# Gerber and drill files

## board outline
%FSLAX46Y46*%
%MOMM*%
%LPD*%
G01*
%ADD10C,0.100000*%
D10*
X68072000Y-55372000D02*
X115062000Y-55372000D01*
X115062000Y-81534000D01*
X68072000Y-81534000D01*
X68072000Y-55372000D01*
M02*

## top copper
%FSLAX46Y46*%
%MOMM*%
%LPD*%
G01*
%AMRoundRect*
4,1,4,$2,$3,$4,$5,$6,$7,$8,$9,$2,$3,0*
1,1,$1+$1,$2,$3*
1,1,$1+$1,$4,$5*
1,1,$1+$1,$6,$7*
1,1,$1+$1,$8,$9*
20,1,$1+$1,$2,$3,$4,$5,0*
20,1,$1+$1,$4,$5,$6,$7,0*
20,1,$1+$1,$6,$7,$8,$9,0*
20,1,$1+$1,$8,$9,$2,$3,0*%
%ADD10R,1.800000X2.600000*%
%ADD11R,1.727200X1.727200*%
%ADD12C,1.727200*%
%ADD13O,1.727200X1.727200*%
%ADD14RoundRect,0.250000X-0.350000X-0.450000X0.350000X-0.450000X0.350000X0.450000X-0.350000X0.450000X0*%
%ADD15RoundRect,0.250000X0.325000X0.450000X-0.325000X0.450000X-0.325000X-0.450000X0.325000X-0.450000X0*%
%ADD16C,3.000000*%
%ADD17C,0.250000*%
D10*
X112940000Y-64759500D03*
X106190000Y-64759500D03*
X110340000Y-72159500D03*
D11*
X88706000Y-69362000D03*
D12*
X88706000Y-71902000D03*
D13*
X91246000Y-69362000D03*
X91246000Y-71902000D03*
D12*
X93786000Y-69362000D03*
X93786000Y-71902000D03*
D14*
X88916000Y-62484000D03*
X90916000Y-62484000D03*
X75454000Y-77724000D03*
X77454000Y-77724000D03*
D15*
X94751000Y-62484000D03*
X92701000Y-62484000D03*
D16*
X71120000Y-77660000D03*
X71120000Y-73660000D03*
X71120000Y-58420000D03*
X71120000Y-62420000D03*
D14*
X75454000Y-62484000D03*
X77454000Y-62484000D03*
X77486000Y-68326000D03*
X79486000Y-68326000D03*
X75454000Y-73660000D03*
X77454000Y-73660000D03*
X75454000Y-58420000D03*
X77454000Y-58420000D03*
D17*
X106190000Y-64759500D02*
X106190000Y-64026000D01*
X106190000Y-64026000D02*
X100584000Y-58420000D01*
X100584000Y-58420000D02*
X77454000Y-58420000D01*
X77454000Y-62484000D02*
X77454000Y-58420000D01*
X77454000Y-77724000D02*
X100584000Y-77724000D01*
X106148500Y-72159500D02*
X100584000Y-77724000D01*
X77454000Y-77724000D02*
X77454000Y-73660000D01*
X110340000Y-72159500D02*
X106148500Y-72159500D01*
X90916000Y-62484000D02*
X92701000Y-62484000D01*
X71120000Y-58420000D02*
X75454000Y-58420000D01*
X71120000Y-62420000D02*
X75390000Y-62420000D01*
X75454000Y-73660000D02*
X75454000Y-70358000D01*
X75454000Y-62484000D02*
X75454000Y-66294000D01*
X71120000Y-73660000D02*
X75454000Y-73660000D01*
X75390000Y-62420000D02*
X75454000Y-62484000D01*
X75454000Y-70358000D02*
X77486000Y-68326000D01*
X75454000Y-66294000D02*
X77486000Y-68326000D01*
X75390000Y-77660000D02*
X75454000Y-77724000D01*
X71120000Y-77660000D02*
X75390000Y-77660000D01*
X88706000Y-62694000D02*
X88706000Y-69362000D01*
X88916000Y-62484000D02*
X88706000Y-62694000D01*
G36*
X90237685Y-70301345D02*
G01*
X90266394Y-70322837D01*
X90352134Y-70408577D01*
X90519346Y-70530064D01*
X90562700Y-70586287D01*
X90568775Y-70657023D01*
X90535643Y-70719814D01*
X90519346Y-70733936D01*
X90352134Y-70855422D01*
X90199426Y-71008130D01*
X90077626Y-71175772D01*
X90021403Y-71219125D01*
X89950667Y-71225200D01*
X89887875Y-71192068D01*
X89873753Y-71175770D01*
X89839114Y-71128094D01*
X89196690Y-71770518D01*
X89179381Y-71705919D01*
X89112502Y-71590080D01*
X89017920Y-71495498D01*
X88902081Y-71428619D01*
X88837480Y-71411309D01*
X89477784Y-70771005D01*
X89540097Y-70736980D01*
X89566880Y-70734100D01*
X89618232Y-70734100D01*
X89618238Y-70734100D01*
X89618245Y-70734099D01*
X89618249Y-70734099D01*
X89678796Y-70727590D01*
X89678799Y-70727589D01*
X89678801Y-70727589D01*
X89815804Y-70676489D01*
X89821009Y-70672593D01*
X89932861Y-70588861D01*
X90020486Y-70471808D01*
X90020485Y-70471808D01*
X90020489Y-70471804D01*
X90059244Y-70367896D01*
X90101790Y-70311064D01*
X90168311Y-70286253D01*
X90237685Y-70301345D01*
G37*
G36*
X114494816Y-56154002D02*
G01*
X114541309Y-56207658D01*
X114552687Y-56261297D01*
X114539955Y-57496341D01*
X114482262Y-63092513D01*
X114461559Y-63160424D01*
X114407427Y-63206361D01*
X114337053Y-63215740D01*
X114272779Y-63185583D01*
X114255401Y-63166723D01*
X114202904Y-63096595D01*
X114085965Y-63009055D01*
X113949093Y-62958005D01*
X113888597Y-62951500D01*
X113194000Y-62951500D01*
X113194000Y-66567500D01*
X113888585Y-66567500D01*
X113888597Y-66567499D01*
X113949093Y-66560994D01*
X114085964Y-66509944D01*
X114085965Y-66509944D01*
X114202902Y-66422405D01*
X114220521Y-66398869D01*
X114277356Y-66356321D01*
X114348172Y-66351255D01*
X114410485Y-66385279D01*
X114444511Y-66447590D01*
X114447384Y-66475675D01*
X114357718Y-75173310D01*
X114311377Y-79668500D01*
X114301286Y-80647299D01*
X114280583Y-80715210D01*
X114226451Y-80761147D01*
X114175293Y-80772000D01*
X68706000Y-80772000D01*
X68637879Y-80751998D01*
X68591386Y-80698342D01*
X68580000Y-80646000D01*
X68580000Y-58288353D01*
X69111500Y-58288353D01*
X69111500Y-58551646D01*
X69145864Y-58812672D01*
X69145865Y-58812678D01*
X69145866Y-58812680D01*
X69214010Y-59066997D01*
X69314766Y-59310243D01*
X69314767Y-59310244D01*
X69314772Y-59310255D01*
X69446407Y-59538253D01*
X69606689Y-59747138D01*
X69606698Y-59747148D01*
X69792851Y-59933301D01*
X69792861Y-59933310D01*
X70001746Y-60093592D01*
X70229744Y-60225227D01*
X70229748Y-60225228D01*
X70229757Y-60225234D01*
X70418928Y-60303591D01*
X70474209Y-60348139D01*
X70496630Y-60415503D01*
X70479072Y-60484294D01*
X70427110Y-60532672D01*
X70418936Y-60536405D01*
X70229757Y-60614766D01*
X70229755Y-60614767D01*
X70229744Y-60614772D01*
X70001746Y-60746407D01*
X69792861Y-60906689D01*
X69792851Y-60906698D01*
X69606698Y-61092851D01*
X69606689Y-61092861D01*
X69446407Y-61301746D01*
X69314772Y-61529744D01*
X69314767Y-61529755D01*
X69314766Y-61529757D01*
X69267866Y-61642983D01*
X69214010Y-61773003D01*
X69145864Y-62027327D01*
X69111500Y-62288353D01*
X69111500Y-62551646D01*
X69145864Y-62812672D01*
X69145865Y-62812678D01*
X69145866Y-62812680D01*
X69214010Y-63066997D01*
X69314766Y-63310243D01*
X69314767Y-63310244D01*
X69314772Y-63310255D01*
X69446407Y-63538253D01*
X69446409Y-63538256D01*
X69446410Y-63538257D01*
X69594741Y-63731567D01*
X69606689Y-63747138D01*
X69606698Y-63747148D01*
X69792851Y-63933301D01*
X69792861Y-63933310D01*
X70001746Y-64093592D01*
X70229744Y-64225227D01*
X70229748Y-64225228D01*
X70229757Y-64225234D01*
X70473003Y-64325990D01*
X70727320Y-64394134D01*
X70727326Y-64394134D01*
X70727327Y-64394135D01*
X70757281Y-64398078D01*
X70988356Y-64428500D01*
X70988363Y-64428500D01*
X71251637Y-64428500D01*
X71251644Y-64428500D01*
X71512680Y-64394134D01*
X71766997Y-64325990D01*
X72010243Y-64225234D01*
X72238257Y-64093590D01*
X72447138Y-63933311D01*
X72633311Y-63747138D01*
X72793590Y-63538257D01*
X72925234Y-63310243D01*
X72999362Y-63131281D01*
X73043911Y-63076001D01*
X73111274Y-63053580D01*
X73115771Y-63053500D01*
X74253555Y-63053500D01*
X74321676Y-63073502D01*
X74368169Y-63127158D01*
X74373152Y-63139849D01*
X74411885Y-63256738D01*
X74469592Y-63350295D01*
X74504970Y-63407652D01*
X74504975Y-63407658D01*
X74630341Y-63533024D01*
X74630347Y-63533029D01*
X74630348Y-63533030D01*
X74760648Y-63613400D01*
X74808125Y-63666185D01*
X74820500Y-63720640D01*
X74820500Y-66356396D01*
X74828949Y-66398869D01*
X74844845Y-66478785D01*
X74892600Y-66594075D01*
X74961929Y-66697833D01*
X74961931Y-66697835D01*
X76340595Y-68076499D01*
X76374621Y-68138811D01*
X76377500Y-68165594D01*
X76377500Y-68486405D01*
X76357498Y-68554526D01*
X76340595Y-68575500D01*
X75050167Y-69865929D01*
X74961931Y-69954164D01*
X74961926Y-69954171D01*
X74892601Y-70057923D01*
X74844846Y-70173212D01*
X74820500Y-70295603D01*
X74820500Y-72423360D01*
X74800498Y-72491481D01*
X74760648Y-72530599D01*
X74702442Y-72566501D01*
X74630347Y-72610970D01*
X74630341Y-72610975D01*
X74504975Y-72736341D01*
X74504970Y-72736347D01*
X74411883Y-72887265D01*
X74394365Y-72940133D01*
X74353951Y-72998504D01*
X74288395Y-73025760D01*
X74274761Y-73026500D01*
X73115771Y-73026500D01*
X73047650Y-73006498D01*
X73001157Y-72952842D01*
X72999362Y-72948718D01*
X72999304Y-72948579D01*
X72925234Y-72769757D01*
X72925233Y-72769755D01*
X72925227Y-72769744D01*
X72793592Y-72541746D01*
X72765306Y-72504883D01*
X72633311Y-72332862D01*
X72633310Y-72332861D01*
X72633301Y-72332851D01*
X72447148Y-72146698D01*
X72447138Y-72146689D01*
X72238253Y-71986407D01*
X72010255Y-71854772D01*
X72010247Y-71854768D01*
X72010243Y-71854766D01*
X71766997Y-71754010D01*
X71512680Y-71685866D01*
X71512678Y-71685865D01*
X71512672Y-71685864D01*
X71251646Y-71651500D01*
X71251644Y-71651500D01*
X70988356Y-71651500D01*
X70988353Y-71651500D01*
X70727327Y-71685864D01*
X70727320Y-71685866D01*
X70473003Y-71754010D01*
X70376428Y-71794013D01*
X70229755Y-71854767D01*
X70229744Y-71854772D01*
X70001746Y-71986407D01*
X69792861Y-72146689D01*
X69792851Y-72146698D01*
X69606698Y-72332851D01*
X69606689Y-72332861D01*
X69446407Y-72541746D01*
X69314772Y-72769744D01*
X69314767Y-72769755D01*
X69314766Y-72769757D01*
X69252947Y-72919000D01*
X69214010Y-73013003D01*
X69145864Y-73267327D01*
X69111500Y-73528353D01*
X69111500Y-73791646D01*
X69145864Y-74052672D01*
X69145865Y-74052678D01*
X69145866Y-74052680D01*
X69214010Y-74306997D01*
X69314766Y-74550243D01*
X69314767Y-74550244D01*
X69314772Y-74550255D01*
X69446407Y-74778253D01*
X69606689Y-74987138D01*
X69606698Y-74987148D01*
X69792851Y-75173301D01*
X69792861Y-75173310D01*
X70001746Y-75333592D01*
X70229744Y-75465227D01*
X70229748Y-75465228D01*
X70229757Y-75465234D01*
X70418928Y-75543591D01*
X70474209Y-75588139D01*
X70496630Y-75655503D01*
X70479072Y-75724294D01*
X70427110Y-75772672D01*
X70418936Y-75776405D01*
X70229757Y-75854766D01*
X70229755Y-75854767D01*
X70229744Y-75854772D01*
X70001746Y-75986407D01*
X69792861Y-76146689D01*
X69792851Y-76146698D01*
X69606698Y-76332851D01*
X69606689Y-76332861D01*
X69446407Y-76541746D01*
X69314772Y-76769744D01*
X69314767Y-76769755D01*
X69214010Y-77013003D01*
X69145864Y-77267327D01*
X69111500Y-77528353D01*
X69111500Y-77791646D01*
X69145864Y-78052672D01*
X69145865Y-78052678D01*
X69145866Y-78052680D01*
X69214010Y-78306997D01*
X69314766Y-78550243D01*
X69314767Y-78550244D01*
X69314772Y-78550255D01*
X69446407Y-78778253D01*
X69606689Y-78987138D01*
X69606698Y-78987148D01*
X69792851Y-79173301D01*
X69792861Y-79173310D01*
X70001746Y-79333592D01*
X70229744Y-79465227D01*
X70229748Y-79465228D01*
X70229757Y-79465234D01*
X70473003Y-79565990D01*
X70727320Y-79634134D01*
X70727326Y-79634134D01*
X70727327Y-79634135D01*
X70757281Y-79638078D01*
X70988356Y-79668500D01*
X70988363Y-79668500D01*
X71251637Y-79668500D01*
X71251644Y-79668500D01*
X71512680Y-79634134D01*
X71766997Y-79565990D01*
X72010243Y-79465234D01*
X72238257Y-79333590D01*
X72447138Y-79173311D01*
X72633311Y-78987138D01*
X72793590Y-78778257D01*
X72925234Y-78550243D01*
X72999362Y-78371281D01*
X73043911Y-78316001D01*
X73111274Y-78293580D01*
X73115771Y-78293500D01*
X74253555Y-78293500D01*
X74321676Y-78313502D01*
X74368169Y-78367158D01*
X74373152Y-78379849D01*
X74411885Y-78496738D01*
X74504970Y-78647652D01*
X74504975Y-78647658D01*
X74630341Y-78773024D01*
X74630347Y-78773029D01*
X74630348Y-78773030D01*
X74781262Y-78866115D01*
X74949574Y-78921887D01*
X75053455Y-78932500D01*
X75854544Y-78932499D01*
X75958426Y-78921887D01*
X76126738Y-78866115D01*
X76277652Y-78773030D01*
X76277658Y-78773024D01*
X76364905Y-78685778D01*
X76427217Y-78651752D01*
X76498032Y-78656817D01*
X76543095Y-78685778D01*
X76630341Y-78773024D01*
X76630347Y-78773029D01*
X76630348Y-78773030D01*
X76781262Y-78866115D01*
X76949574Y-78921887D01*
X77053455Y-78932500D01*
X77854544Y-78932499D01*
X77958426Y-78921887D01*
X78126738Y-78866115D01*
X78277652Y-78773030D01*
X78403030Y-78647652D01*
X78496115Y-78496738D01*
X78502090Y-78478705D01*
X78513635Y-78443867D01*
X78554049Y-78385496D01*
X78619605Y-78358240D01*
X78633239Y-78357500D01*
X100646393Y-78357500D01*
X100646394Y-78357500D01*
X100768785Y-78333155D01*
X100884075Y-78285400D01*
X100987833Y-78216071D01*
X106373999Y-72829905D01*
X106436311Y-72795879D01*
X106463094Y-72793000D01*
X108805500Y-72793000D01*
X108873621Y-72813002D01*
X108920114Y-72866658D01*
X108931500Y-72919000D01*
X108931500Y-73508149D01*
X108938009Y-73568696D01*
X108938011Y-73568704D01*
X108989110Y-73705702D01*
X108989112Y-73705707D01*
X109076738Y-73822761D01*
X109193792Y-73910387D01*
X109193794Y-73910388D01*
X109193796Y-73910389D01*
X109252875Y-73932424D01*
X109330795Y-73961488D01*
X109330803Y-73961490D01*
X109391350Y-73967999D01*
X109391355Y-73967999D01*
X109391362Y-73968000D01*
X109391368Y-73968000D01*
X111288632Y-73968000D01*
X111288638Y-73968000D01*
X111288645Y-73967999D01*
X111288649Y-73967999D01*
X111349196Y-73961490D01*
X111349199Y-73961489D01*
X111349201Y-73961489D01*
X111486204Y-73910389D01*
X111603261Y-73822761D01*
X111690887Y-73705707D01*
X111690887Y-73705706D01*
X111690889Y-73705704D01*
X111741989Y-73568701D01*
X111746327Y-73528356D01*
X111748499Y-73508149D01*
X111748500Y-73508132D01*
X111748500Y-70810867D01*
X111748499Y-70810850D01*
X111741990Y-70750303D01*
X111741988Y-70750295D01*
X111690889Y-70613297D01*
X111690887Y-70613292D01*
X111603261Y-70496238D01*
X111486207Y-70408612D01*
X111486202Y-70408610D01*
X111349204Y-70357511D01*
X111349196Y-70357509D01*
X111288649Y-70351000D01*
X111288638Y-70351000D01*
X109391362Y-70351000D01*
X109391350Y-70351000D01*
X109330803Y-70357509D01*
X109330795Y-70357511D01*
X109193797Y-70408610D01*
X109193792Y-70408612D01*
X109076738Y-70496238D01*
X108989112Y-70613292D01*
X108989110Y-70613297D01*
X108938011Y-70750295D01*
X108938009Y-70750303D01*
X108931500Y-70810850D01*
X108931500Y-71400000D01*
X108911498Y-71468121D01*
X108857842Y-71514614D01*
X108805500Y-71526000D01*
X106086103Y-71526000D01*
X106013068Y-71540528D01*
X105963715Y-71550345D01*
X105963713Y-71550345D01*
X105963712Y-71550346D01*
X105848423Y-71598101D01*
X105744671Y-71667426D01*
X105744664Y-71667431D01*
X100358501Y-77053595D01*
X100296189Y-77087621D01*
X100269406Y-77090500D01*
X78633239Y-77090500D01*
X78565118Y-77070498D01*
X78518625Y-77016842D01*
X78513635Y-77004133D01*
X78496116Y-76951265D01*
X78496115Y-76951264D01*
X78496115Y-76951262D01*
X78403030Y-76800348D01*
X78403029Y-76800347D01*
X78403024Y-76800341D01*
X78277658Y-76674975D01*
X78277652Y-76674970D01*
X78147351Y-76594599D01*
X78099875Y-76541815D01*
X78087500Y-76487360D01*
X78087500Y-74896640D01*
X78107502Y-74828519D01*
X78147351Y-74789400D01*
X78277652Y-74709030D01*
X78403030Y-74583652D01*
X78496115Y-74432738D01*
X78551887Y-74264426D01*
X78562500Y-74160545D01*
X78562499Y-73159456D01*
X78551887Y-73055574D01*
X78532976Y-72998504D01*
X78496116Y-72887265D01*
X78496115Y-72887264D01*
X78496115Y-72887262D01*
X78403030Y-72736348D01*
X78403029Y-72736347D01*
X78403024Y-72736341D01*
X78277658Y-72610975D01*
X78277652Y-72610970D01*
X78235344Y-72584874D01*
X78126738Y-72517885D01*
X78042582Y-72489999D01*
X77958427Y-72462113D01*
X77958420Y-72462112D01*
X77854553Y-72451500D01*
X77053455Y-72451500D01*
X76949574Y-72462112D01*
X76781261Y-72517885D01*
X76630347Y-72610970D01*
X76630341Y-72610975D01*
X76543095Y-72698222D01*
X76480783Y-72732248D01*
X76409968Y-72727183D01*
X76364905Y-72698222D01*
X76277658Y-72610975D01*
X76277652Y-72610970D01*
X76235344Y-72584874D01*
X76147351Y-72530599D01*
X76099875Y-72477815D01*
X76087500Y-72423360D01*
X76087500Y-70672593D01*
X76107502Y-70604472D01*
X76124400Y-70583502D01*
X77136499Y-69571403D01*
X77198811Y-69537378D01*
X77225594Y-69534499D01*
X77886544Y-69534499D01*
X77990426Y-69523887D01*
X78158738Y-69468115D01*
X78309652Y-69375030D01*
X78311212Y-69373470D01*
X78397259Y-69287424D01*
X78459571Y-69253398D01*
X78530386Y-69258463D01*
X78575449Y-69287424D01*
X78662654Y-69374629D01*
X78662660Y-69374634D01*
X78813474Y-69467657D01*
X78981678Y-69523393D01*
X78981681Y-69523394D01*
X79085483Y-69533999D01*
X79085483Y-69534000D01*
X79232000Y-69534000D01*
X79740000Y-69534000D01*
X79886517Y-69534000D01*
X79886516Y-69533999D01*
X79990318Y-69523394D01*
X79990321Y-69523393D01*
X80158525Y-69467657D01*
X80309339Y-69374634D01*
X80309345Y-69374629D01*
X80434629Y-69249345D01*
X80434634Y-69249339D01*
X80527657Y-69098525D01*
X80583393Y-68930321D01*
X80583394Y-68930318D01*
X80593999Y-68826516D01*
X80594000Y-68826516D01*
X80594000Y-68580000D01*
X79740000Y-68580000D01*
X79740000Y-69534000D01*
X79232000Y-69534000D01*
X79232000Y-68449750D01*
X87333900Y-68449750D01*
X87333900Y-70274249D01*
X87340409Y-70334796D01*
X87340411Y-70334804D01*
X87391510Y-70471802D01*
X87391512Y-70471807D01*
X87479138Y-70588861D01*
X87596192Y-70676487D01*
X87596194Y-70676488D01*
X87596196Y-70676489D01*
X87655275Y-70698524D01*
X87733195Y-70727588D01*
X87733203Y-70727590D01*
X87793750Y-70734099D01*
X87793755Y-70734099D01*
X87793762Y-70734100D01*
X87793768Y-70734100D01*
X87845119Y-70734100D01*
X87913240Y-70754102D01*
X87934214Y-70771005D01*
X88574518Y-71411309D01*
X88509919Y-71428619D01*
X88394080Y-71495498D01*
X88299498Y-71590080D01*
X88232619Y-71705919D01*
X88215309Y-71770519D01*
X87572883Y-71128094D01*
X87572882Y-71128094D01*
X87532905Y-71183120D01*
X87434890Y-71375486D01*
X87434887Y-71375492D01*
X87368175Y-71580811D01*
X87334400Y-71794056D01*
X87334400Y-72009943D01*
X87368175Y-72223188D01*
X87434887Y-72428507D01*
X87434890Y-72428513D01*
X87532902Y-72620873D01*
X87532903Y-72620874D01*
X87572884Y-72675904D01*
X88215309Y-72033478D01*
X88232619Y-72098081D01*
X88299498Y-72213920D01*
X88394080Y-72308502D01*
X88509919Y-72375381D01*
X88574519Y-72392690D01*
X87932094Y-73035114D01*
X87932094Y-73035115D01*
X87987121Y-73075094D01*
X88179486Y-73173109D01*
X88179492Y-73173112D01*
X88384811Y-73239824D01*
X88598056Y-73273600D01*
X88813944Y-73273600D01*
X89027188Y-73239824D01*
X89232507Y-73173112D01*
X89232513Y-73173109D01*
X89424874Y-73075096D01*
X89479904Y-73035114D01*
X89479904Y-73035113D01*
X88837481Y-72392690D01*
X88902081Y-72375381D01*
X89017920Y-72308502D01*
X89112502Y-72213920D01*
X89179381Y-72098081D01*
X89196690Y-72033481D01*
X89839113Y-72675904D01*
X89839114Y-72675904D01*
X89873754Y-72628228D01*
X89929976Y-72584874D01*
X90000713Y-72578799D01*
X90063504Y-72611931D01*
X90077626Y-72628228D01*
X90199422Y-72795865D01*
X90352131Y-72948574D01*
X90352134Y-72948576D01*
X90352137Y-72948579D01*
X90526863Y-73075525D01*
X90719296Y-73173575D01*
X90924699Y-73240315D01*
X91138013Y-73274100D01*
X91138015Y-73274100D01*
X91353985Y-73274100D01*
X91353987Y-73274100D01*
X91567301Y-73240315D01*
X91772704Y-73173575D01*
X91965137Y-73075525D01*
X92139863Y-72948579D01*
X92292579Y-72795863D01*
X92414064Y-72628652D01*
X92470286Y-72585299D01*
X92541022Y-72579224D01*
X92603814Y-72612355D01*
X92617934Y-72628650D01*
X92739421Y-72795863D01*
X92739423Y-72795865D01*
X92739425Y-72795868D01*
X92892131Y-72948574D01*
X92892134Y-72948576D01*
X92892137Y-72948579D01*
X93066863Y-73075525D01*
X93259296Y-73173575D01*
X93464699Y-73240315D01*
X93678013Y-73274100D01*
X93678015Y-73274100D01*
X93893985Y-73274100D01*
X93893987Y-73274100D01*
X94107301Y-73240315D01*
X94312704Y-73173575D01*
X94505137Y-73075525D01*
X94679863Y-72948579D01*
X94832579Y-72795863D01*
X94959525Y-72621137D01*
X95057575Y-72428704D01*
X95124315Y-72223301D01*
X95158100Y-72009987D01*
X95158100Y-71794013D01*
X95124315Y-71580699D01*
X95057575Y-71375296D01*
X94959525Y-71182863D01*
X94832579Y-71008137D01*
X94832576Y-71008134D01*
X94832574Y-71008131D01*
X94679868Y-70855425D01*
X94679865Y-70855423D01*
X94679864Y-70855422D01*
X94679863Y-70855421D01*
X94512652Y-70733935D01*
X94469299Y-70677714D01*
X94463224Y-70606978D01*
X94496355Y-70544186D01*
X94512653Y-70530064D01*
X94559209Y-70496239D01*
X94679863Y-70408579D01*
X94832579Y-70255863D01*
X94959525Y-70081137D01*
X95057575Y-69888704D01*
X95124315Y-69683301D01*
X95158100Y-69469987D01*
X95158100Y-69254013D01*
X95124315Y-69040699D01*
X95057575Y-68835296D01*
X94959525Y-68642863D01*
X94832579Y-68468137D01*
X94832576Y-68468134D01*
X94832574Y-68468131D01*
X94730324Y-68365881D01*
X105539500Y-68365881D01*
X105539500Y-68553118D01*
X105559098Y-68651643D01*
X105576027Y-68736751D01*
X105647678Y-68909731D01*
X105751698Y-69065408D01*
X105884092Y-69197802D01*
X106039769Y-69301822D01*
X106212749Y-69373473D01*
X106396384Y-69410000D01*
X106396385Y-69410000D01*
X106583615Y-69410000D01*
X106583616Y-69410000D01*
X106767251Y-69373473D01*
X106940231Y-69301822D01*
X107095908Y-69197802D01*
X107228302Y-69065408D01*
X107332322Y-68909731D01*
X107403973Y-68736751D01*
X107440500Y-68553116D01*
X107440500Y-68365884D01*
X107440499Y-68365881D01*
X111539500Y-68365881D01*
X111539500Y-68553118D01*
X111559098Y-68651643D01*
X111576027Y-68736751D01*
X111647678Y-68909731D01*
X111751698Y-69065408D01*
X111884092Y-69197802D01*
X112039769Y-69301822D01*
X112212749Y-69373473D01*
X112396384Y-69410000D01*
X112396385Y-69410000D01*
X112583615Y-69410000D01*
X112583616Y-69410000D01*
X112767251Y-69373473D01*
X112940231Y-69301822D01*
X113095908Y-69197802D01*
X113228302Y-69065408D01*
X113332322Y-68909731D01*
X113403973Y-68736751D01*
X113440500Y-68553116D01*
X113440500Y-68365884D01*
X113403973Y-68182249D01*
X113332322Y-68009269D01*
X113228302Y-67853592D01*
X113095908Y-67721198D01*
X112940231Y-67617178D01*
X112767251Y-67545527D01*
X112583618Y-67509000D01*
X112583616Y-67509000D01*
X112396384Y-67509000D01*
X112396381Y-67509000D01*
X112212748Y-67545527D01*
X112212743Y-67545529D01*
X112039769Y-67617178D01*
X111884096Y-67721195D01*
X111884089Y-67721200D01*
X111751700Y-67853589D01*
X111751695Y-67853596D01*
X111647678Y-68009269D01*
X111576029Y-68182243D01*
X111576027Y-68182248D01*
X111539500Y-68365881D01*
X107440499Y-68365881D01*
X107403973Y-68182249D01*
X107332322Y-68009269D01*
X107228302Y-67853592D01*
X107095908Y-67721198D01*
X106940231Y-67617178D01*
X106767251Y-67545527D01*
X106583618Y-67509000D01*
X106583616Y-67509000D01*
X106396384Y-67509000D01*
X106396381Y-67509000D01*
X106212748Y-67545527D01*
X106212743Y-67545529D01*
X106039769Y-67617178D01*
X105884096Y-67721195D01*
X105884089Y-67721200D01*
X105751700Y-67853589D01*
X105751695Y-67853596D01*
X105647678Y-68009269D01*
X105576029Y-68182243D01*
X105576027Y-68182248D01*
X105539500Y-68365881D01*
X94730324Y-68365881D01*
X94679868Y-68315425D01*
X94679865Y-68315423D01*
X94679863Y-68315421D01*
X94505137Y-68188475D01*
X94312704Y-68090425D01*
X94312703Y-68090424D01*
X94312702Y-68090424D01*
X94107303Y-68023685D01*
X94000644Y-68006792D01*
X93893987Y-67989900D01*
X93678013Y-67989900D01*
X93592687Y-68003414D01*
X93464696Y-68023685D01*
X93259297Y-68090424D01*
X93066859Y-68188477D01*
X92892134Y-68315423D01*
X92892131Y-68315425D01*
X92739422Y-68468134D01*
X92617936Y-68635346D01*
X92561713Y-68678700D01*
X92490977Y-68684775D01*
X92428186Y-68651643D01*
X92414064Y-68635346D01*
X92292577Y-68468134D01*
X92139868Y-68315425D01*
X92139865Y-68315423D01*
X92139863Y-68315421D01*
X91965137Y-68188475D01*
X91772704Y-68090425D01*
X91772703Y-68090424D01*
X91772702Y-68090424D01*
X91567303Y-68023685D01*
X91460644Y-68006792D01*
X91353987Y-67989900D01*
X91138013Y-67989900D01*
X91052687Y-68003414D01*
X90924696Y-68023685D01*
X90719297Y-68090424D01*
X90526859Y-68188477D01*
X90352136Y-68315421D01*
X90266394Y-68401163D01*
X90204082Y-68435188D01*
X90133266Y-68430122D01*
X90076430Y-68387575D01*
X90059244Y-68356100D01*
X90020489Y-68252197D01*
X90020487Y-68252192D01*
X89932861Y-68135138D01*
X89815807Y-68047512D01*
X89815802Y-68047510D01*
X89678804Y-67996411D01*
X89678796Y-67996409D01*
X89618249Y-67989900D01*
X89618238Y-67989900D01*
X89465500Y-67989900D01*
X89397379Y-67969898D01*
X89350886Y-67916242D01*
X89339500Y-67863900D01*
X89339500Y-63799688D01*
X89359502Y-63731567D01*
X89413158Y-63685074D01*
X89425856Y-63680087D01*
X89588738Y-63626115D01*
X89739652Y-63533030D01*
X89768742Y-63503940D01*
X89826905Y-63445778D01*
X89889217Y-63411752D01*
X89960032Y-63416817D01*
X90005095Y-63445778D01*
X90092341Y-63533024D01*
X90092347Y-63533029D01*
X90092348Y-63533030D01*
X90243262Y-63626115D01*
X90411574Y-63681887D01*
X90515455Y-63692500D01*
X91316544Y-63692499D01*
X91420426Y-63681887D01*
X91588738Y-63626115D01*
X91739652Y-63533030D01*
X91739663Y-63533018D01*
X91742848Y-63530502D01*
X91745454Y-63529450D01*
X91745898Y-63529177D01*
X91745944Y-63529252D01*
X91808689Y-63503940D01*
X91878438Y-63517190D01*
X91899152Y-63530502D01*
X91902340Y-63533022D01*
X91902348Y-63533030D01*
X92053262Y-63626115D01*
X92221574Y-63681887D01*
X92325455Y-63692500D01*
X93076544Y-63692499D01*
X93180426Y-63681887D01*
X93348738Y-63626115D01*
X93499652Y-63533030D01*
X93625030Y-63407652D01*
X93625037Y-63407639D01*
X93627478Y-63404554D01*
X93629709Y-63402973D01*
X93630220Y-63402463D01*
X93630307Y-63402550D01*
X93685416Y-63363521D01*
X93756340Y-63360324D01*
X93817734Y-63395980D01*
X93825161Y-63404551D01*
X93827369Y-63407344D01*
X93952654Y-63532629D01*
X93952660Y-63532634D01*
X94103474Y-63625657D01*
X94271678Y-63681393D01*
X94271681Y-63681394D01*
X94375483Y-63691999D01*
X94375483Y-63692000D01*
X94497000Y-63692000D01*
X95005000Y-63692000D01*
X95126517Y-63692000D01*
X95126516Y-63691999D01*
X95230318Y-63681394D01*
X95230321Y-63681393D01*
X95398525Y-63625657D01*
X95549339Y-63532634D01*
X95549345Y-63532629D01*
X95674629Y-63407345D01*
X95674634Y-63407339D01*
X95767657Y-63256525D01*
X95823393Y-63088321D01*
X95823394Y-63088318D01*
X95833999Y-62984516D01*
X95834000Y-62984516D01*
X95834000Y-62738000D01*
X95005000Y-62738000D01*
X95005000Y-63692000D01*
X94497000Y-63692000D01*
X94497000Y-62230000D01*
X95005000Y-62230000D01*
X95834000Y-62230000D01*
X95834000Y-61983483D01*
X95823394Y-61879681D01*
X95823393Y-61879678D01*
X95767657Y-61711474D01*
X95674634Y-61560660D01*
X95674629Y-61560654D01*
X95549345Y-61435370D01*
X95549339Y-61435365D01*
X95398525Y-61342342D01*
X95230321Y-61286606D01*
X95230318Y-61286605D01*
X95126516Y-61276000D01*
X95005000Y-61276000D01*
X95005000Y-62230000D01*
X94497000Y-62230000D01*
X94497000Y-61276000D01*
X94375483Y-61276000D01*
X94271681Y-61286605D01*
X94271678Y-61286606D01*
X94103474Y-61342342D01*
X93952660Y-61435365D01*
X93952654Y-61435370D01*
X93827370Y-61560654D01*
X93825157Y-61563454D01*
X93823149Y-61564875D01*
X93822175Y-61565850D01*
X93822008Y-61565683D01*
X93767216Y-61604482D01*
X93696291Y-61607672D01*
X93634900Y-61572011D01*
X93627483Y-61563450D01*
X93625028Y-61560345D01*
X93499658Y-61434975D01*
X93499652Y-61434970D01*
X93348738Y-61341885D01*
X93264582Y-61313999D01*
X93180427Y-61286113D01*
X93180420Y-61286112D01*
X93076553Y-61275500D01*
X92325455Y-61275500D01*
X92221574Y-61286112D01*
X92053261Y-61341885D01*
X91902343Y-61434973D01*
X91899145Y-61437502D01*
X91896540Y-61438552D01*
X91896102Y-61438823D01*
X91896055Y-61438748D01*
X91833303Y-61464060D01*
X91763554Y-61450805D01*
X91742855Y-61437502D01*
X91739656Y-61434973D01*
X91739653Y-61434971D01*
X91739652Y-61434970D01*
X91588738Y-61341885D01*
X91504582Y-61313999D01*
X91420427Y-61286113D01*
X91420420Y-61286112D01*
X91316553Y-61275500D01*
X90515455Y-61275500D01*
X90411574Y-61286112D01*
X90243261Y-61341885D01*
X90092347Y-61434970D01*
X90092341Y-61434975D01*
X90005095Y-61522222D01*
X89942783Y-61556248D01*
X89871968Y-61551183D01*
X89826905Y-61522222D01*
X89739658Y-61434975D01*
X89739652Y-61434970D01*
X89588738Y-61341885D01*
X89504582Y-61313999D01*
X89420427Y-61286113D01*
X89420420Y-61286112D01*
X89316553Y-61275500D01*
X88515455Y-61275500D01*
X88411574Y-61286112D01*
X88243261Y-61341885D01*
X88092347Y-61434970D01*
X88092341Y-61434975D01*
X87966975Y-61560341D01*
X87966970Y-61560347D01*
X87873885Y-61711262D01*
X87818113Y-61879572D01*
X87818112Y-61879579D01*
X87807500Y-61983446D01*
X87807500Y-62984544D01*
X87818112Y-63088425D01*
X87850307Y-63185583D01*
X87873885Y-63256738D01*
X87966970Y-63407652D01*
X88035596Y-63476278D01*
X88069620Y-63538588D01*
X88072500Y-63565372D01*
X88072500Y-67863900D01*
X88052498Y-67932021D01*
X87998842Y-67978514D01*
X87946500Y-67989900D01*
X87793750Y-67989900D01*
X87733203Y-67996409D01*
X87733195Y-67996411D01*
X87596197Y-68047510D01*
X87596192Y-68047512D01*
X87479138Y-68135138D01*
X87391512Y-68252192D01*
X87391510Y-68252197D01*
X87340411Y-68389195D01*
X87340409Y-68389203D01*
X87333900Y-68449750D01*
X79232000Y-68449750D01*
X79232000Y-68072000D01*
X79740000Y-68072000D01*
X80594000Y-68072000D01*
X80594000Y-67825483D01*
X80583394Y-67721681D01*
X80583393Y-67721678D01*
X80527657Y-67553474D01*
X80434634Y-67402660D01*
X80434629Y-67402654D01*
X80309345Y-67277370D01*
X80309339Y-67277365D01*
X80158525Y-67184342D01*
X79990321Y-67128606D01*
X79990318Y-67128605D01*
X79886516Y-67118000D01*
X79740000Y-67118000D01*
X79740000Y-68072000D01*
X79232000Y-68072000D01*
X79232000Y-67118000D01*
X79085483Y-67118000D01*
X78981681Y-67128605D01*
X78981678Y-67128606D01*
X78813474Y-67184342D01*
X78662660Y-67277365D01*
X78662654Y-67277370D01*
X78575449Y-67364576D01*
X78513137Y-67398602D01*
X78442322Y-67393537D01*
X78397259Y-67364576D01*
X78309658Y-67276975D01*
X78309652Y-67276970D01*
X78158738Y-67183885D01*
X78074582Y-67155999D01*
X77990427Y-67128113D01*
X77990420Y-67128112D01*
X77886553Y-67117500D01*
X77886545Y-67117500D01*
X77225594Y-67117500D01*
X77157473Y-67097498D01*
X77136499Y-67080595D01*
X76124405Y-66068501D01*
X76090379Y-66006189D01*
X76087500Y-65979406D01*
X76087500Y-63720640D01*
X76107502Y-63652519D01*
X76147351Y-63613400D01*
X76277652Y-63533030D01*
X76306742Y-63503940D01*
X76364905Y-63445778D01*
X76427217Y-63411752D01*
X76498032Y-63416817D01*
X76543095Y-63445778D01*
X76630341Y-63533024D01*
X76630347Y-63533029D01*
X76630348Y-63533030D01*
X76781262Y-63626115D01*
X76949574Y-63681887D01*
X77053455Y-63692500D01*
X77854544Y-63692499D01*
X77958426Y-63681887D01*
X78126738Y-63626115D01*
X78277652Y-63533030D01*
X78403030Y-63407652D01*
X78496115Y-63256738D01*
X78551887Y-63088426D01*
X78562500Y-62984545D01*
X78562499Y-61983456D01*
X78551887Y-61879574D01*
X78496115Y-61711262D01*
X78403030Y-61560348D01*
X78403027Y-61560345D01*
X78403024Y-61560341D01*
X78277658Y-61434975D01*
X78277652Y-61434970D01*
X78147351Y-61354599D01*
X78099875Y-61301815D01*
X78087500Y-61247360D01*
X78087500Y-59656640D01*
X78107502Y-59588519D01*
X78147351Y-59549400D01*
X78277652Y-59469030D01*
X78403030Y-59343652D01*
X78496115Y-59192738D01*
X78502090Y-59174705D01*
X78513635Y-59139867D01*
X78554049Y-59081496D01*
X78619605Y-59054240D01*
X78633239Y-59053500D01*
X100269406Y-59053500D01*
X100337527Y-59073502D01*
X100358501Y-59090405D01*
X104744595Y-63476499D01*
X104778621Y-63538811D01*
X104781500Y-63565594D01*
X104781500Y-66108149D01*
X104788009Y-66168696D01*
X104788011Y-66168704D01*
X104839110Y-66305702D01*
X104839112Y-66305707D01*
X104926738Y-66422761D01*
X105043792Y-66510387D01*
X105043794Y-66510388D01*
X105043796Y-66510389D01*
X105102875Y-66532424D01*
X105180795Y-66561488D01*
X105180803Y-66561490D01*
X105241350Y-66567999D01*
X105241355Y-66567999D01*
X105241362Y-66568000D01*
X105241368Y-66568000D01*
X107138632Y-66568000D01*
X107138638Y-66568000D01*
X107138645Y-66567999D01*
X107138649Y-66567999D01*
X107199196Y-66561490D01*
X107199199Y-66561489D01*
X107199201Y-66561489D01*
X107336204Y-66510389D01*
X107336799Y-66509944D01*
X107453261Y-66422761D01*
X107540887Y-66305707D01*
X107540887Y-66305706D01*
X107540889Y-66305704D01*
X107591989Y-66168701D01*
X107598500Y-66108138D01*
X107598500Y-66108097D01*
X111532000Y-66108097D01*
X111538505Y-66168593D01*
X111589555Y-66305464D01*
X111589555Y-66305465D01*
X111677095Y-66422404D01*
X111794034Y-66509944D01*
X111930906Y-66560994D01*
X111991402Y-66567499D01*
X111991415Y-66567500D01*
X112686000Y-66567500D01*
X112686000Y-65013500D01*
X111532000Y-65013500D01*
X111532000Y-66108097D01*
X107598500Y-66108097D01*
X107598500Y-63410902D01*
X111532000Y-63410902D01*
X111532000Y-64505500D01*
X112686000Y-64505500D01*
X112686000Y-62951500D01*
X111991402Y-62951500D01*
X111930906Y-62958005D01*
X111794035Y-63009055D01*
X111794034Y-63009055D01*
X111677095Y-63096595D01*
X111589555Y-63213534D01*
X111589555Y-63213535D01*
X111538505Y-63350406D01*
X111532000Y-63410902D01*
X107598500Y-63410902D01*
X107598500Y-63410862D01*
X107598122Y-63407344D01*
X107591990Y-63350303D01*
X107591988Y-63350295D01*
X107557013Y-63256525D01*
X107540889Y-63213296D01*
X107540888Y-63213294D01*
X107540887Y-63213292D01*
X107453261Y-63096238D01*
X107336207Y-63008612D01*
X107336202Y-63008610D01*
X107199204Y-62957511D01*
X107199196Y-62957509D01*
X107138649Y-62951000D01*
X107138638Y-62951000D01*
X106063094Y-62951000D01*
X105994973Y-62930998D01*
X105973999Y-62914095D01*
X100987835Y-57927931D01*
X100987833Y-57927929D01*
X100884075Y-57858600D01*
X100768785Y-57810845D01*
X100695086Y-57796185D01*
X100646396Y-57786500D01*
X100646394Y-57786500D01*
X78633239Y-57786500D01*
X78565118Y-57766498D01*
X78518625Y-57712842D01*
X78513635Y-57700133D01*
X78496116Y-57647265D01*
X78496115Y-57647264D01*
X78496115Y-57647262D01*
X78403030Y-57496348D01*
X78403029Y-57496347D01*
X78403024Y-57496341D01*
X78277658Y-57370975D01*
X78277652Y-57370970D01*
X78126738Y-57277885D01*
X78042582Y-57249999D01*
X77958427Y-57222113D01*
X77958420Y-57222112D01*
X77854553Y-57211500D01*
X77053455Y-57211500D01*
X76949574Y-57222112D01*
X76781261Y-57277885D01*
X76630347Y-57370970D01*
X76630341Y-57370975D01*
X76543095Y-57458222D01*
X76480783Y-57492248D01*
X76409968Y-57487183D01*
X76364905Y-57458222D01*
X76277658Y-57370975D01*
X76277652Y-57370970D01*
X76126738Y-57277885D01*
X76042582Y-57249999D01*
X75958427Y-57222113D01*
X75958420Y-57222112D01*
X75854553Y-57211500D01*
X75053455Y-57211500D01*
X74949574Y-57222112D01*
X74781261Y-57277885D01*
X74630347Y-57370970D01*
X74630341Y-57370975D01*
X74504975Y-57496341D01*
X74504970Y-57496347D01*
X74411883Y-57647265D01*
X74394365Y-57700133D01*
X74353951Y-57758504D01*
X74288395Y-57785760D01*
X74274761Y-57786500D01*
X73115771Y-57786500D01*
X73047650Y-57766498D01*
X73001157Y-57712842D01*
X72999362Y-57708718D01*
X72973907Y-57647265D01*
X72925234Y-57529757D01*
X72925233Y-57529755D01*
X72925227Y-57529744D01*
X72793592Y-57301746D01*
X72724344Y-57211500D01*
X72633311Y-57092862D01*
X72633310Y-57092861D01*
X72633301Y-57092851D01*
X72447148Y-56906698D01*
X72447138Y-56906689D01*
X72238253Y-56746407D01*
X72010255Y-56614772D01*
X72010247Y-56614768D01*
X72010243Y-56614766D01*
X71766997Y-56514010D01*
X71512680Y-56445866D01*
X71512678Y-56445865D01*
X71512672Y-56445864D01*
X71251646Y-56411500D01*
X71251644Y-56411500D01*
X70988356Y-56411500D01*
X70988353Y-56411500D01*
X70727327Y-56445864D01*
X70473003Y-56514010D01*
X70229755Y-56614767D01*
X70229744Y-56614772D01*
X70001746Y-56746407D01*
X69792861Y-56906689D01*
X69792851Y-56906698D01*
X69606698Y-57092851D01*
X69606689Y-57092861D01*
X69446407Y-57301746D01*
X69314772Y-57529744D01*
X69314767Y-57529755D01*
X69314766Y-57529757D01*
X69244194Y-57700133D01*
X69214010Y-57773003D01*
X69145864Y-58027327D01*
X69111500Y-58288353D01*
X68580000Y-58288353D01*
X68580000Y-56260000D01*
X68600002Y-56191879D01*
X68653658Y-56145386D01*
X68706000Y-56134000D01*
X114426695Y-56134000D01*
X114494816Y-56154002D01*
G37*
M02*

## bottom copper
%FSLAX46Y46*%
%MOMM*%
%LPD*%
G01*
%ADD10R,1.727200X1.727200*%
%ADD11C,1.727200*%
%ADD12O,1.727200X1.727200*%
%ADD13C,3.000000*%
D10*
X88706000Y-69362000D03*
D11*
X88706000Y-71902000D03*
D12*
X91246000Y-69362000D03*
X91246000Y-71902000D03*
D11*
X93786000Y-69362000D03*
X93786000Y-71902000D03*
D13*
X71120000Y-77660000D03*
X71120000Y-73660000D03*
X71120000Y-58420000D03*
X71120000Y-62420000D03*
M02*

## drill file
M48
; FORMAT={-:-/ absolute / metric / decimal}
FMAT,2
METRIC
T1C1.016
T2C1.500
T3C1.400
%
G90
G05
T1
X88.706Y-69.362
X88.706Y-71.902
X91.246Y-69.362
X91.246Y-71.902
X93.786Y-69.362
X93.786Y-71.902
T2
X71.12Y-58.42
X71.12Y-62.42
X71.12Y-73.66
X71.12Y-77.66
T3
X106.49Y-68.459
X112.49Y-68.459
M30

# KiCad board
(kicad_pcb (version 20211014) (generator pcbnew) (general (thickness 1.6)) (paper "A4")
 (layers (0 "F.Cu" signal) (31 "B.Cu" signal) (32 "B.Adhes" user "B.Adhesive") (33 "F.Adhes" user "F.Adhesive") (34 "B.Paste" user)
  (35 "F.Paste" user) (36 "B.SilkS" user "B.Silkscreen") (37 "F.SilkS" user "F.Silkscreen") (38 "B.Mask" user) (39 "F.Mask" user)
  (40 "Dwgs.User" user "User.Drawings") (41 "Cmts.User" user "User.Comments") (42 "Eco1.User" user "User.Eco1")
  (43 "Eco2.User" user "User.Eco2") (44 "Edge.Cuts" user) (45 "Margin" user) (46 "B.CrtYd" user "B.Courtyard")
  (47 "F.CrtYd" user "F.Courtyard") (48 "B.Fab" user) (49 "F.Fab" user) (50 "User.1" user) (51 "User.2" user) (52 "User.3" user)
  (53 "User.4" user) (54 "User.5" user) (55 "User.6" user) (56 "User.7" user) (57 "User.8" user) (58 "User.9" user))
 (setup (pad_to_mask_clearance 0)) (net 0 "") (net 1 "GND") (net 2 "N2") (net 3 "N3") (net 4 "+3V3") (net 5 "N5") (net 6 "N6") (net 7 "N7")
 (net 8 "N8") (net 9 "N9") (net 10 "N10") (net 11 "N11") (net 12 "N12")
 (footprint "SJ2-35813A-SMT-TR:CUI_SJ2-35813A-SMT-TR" (layer "F.Cu") (at 109.24 68.4595 180)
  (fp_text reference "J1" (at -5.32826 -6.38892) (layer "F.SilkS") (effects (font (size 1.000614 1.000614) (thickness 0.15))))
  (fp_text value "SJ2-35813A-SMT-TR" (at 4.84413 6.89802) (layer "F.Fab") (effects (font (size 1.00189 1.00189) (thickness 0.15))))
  (pad "" np_thru_hole circle locked (at -3.25 0 180) (size 1.4 1.4) (drill 1.4) (layers *.Cu *.Mask))
  (pad "" np_thru_hole circle locked (at 2.75 0 180) (size 1.4 1.4) (drill 1.4) (layers *.Cu *.Mask))
  (pad "1" smd rect locked (at -3.7 3.7 180) (size 1.8 2.6) (layers "F.Cu" "F.Paste" "F.Mask") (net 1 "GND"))
  (pad "2" smd rect locked (at 3.05 3.7 180) (size 1.8 2.6) (layers "F.Cu" "F.Paste" "F.Mask") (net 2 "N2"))
  (pad "3" smd rect locked (at -1.1 -3.7 180) (size 1.8 2.6) (layers "F.Cu" "F.Paste" "F.Mask") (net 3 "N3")))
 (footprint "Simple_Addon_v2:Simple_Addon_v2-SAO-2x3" (layer "F.Cu") (at 91.186 70.612)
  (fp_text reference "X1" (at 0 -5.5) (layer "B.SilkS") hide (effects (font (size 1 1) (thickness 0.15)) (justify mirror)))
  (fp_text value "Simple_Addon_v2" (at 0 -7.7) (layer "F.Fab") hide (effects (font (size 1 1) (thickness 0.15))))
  (pad "1" thru_hole rect (at -2.48 -1.25 270) (size 1.7272 1.7272) (drill 1.016) (layers *.Cu *.Mask) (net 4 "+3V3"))
  (pad "2" thru_hole circle (at -2.48 1.29 270) (size 1.7272 1.7272) (drill 1.016) (layers *.Cu *.Mask) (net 1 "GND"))
  (pad "3" thru_hole oval (at 0.06 -1.25 270) (size 1.7272 1.7272) (drill 1.016) (layers *.Cu *.Mask) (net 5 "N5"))
  (pad "4" thru_hole oval (at 0.06 1.29 270) (size 1.7272 1.7272) (drill 1.016) (layers *.Cu *.Mask) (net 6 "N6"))
  (pad "5" thru_hole circle (at 2.6 -1.25 270) (size 1.7272 1.7272) (drill 1.016) (layers *.Cu *.Mask) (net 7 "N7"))
  (pad "6" thru_hole circle (at 2.6 1.29 270) (size 1.7272 1.7272) (drill 1.016) (layers *.Cu *.Mask) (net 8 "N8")))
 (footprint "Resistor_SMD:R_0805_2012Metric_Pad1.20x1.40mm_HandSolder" (layer "F.Cu") (at 89.916 62.484)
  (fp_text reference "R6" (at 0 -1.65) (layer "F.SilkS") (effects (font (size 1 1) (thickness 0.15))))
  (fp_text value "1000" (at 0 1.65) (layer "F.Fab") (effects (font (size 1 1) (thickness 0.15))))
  (pad "1" smd roundrect (at -1 0) (size 1.2 1.4) (layers "F.Cu" "F.Paste" "F.Mask") (roundrect_rratio 0.2083333333) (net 4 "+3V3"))
  (pad "2" smd roundrect (at 1 0) (size 1.2 1.4) (layers "F.Cu" "F.Paste" "F.Mask") (roundrect_rratio 0.2083333333) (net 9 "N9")))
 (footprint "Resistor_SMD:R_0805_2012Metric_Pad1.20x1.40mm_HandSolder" (layer "F.Cu") (at 76.454 77.724)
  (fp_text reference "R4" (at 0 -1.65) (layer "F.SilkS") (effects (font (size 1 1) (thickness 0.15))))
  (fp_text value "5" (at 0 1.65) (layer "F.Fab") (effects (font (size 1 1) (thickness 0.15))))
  (pad "1" smd roundrect (at -1 0) (size 1.2 1.4) (layers "F.Cu" "F.Paste" "F.Mask") (roundrect_rratio 0.2083333333) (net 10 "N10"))
  (pad "2" smd roundrect (at 1 0) (size 1.2 1.4) (layers "F.Cu" "F.Paste" "F.Mask") (roundrect_rratio 0.2083333333) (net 3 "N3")))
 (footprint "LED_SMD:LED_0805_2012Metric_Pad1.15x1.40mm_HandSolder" (layer "F.Cu") (at 93.726 62.484 180)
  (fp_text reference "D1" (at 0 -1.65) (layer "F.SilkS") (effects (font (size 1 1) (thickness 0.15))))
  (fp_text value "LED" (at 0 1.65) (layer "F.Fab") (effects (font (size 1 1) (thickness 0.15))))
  (pad "1" smd roundrect (at -1.025 0 180) (size 1.15 1.4) (layers "F.Cu" "F.Paste" "F.Mask") (roundrect_rratio 0.2173913043) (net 1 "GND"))
  (pad "2" smd roundrect (at 1.025 0 180) (size 1.15 1.4) (layers "F.Cu" "F.Paste" "F.Mask") (roundrect_rratio 0.2173913043) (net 9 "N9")))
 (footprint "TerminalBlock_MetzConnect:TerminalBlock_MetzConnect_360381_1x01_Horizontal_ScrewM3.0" (layer "F.Cu") (at 71.12 73.66 -90)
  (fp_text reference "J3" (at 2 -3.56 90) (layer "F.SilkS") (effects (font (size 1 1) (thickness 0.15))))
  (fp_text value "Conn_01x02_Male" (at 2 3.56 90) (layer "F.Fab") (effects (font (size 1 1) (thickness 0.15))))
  (pad "1" thru_hole circle (at 4 0 270) (size 3 3) (drill 1.5) (layers *.Cu *.Mask) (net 10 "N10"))
  (pad "2" thru_hole circle (at 0 0 270) (size 3 3) (drill 1.5) (layers *.Cu *.Mask) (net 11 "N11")))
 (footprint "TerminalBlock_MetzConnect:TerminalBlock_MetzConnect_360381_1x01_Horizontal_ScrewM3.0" (layer "F.Cu") (at 71.12 58.42 -90)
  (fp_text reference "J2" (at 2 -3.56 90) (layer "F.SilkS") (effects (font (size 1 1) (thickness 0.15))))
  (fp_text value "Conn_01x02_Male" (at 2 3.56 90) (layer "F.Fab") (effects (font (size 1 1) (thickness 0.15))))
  (pad "1" thru_hole circle (at 0 0 270) (size 3 3) (drill 1.5) (layers *.Cu *.Mask) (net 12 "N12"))
  (pad "2" thru_hole circle (at 4 0 270) (size 3 3) (drill 1.5) (layers *.Cu *.Mask) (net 11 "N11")))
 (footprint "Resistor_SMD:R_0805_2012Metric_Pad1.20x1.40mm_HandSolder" (layer "F.Cu") (at 76.454 62.484)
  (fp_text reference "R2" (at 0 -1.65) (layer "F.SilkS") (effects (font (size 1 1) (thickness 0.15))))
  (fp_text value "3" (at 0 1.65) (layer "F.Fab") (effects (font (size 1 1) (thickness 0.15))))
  (pad "1" smd roundrect (at -1 0) (size 1.2 1.4) (layers "F.Cu" "F.Paste" "F.Mask") (roundrect_rratio 0.2083333333) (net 11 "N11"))
  (pad "2" smd roundrect (at 1 0) (size 1.2 1.4) (layers "F.Cu" "F.Paste" "F.Mask") (roundrect_rratio 0.2083333333) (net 2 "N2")))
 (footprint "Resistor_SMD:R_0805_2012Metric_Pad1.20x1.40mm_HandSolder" (layer "F.Cu") (at 78.486 68.326)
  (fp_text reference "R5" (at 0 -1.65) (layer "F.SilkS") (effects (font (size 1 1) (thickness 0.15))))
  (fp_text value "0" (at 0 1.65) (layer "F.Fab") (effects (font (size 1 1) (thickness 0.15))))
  (pad "1" smd roundrect (at -1 0) (size 1.2 1.4) (layers "F.Cu" "F.Paste" "F.Mask") (roundrect_rratio 0.2083333333) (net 11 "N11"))
  (pad "2" smd roundrect (at 1 0) (size 1.2 1.4) (layers "F.Cu" "F.Paste" "F.Mask") (roundrect_rratio 0.2083333333) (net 1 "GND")))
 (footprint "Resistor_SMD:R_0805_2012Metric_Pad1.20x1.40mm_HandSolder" (layer "F.Cu") (at 76.454 73.66)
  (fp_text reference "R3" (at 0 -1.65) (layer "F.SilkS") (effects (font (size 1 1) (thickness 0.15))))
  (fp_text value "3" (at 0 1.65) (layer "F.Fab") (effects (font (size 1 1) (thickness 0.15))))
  (pad "1" smd roundrect (at -1 0) (size 1.2 1.4) (layers "F.Cu" "F.Paste" "F.Mask") (roundrect_rratio 0.2083333333) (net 11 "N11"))
  (pad "2" smd roundrect (at 1 0) (size 1.2 1.4) (layers "F.Cu" "F.Paste" "F.Mask") (roundrect_rratio 0.2083333333) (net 3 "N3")))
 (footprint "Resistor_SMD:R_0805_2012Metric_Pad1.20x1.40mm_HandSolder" (layer "F.Cu") (at 76.454 58.42)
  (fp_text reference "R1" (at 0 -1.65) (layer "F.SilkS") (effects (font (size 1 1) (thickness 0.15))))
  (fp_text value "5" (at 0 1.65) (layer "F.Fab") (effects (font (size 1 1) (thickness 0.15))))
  (pad "1" smd roundrect (at -1 0) (size 1.2 1.4) (layers "F.Cu" "F.Paste" "F.Mask") (roundrect_rratio 0.2083333333) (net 12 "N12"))
  (pad "2" smd roundrect (at 1 0) (size 1.2 1.4) (layers "F.Cu" "F.Paste" "F.Mask") (roundrect_rratio 0.2083333333) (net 2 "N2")))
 (gr_rect (start 68.072 55.372) (end 115.062 81.534) (layer "Edge.Cuts") (width 0.1) (fill none))
 (segment (start 106.19 64.7595) (end 106.19 64.026) (width 0.25) (layer "F.Cu") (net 2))
 (segment (start 106.19 64.026) (end 100.584 58.42) (width 0.25) (layer "F.Cu") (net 2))
 (segment (start 100.584 58.42) (end 77.454 58.42) (width 0.25) (layer "F.Cu") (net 2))
 (segment (start 77.454 62.484) (end 77.454 58.42) (width 0.25) (layer "F.Cu") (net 2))
 (segment (start 77.454 77.724) (end 100.584 77.724) (width 0.25) (layer "F.Cu") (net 3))
 (segment (start 106.1485 72.1595) (end 100.584 77.724) (width 0.25) (layer "F.Cu") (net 3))
 (segment (start 77.454 77.724) (end 77.454 73.66) (width 0.25) (layer "F.Cu") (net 3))
 (segment (start 110.34 72.1595) (end 106.1485 72.1595) (width 0.25) (layer "F.Cu") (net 3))
 (segment (start 90.916 62.484) (end 92.701 62.484) (width 0.25) (layer "F.Cu") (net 9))
 (segment (start 71.12 58.42) (end 75.454 58.42) (width 0.25) (layer "F.Cu") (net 12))
 (segment (start 71.12 62.42) (end 75.39 62.42) (width 0.25) (layer "F.Cu") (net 11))
 (segment (start 75.454 73.66) (end 75.454 70.358) (width 0.25) (layer "F.Cu") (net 11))
 (segment (start 75.454 62.484) (end 75.454 66.294) (width 0.25) (layer "F.Cu") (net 11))
 (segment (start 71.12 73.66) (end 75.454 73.66) (width 0.25) (layer "F.Cu") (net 11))
 (segment (start 75.39 62.42) (end 75.454 62.484) (width 0.25) (layer "F.Cu") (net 11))
 (segment (start 75.454 70.358) (end 77.486 68.326) (width 0.25) (layer "F.Cu") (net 11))
 (segment (start 75.454 66.294) (end 77.486 68.326) (width 0.25) (layer "F.Cu") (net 11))
 (segment (start 75.39 77.66) (end 75.454 77.724) (width 0.25) (layer "F.Cu") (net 10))
 (segment (start 71.12 77.66) (end 75.39 77.66) (width 0.25) (layer "F.Cu") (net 10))
 (segment (start 88.706 62.694) (end 88.706 69.362) (width 0.25) (layer "F.Cu") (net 4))
 (segment (start 88.916 62.484) (end 88.706 62.694) (width 0.25) (layer "F.Cu") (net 4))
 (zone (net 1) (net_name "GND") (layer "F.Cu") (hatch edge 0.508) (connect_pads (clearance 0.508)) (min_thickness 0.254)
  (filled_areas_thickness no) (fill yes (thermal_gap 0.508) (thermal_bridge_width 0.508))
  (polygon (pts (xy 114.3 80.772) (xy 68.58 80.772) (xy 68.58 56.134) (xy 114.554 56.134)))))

